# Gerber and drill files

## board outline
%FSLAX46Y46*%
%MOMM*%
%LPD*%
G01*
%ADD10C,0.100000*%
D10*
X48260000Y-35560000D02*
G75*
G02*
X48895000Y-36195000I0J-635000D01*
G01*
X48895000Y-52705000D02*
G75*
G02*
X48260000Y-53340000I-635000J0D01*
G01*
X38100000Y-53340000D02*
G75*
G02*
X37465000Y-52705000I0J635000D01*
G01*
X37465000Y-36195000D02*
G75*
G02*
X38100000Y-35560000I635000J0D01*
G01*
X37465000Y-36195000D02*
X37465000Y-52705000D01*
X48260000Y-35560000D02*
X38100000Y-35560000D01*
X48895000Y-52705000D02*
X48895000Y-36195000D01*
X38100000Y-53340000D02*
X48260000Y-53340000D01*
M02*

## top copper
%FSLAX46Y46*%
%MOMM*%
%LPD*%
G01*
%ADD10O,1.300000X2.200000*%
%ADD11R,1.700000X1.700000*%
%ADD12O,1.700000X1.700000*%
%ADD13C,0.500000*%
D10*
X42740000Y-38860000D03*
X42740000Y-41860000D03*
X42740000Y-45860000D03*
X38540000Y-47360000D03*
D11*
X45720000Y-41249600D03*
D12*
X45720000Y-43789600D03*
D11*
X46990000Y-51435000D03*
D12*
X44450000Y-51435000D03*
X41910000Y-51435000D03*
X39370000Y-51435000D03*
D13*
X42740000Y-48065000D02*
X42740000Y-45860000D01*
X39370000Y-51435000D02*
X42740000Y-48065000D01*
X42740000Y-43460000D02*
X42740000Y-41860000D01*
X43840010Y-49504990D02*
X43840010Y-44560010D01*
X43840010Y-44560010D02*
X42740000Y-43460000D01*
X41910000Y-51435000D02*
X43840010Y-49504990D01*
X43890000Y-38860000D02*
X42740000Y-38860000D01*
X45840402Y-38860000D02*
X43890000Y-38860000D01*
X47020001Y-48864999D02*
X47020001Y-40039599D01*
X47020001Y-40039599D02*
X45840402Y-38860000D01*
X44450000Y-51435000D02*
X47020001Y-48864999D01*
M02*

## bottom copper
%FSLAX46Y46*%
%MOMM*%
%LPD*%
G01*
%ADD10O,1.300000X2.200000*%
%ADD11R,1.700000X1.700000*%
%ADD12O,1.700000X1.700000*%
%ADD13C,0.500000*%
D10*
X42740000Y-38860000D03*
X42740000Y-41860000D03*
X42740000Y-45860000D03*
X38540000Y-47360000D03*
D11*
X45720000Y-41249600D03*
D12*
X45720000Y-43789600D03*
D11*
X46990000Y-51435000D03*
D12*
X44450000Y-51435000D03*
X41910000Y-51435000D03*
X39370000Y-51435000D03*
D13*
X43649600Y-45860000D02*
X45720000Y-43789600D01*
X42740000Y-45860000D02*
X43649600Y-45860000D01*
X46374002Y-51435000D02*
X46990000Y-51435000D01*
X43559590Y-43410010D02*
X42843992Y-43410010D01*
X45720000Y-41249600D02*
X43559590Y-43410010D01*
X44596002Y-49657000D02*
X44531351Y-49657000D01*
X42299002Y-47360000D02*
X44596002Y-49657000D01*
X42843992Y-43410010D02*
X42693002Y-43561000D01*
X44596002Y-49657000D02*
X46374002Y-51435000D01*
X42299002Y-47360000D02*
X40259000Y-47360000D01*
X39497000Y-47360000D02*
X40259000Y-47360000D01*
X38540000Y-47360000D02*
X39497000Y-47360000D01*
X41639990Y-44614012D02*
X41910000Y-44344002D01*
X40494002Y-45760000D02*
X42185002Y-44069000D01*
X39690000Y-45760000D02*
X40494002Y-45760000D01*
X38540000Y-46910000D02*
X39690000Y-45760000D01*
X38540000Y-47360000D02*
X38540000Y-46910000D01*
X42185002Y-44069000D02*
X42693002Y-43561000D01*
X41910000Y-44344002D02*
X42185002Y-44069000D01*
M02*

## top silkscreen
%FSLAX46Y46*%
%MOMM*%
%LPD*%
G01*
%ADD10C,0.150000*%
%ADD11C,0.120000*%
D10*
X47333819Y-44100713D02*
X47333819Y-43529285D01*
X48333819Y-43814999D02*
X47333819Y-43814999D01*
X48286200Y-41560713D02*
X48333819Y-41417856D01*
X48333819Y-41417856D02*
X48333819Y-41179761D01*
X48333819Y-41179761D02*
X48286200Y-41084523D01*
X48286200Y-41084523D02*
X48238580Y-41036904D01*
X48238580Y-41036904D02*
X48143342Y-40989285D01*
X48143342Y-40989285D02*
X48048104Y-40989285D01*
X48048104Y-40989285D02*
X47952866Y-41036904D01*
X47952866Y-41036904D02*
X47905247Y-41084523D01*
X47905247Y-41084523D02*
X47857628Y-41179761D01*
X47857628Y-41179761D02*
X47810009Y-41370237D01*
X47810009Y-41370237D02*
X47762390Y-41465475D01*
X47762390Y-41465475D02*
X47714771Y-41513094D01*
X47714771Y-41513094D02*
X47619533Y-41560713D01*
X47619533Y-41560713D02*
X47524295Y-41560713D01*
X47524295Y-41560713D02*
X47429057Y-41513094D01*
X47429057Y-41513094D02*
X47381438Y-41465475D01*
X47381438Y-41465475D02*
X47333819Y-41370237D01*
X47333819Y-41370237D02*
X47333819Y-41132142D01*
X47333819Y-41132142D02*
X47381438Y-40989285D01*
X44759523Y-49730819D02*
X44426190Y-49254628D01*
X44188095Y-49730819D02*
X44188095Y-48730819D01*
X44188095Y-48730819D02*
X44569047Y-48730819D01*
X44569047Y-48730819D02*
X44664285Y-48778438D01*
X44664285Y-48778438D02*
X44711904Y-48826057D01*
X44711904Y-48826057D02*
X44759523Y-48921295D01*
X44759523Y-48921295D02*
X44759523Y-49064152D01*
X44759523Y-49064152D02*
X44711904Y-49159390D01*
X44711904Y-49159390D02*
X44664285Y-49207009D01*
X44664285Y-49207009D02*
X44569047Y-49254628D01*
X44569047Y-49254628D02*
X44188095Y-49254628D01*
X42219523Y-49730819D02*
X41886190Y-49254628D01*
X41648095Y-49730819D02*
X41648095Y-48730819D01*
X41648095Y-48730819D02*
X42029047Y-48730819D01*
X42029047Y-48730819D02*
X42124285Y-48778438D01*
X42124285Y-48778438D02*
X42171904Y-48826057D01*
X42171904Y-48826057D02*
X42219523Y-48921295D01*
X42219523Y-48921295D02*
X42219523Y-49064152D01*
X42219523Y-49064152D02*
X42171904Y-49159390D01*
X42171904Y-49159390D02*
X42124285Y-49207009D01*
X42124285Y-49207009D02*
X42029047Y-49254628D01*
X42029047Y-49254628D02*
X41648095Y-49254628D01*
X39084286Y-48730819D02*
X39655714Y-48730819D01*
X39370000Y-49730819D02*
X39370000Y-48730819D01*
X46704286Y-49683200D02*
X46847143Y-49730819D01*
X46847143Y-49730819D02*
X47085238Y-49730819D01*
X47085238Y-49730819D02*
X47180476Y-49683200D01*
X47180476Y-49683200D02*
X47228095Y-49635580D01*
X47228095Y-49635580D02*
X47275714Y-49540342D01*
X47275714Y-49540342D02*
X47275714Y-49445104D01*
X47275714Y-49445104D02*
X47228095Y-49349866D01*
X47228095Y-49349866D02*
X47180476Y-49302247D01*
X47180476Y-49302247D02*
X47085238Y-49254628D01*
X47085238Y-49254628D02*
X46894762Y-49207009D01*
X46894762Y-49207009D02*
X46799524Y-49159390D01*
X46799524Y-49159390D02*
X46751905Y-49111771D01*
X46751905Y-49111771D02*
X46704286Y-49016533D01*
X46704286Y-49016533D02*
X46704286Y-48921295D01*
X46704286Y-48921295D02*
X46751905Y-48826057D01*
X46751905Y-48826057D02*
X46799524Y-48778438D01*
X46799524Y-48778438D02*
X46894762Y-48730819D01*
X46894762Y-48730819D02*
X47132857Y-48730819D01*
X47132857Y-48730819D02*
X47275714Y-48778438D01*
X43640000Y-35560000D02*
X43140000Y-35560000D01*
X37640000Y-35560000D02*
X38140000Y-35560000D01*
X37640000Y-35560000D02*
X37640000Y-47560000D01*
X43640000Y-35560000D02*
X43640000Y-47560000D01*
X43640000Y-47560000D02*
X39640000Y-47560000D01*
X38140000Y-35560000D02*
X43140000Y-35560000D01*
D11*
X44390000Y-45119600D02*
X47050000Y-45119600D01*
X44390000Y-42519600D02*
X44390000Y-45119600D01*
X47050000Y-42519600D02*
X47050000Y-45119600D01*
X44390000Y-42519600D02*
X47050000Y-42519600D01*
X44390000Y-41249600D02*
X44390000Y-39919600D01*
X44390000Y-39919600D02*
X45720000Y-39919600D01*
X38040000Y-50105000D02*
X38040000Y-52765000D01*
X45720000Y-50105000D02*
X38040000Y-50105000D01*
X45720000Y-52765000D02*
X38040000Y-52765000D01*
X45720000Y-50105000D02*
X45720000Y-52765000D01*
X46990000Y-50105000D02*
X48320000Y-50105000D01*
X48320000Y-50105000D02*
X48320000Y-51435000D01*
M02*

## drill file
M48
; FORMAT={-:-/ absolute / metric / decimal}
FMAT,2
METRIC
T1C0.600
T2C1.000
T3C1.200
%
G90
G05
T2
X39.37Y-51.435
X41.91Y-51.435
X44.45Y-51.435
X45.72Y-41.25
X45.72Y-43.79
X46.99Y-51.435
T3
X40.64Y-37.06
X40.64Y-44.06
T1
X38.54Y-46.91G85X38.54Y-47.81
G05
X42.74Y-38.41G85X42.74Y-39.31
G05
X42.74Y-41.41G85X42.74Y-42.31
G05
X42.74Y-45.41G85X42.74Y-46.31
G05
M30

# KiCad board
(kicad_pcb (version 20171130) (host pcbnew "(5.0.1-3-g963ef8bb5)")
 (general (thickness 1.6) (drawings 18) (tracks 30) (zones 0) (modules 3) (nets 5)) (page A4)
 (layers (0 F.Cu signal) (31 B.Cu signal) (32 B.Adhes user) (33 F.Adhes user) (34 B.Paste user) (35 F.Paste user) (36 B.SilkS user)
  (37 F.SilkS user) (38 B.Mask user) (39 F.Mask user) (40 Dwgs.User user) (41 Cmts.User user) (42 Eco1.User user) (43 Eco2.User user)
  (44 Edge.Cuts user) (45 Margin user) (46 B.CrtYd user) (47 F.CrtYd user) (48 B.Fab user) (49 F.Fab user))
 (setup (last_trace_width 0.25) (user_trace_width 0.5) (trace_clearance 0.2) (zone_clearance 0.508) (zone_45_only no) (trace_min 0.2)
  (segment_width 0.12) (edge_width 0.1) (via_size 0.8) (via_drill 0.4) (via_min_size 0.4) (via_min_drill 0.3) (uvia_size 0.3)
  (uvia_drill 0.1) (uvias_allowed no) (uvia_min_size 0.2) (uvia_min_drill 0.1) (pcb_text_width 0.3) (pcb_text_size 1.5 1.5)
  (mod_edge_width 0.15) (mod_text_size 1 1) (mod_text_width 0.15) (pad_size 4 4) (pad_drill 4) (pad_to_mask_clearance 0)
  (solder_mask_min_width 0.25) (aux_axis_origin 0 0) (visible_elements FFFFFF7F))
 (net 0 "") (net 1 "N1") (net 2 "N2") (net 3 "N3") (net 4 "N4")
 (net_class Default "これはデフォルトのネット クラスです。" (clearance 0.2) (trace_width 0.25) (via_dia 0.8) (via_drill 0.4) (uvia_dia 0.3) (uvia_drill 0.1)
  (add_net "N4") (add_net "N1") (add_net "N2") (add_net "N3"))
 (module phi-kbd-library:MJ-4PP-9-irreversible (layer F.Cu) (at 40.64 35.56 270)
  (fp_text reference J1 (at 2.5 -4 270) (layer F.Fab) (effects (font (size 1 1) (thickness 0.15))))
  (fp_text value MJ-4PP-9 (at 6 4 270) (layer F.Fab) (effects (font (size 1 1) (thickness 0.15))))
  (fp_line (start 0 -3) (end 0 -2.5) (layer F.SilkS) (width 0.15))
  (fp_line (start 0 3) (end 0 2.5) (layer F.SilkS) (width 0.15))
  (fp_line (start 0 3) (end 12 3) (layer F.SilkS) (width 0.15))
  (fp_line (start 0 -3) (end 12 -3) (layer F.SilkS) (width 0.15))
  (fp_line (start 12 -3) (end 12 1) (layer F.SilkS) (width 0.15))
  (fp_line (start 0 2.5) (end 0 -2.5) (layer F.SilkS) (width 0.15))
  (pad "" np_thru_hole circle (at 1.5 0 270) (size 1.2 1.2) (drill 1.2) (layers *.Cu *.Mask))
  (pad "" np_thru_hole circle (at 8.5 0 270) (size 1.2 1.2) (drill 1.2) (layers *.Cu *.Mask))
  (pad B thru_hole oval (at 3.3 -2.1 270) (size 2.2 1.3) (drill oval 1.5 0.6) (layers *.Cu *.Mask) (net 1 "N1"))
  (pad C thru_hole oval (at 6.3 -2.1 270) (size 2.2 1.3) (drill oval 1.5 0.6) (layers *.Cu *.Mask) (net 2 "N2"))
  (pad D thru_hole oval (at 10.3 -2.1 270) (size 2.2 1.3) (drill oval 1.5 0.6) (layers *.Cu *.Mask) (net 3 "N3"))
  (pad A thru_hole oval (at 11.8 2.1 270) (size 2.2 1.3) (drill oval 1.5 0.6) (layers *.Cu *.Mask) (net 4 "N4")))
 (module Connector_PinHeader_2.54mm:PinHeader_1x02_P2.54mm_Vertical (layer F.Cu) (at 45.72 41.2496)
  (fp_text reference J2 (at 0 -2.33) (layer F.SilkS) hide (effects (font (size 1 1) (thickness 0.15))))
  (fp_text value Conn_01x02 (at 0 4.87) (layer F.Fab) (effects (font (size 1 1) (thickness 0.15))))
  (fp_line (start -1.33 3.87) (end 1.33 3.87) (layer F.SilkS) (width 0.12))
  (fp_line (start -1.33 1.27) (end -1.33 3.87) (layer F.SilkS) (width 0.12))
  (fp_line (start 1.33 1.27) (end 1.33 3.87) (layer F.SilkS) (width 0.12))
  (fp_line (start -1.33 1.27) (end 1.33 1.27) (layer F.SilkS) (width 0.12))
  (fp_line (start -1.33 0) (end -1.33 -1.33) (layer F.SilkS) (width 0.12))
  (fp_line (start -1.33 -1.33) (end 0 -1.33) (layer F.SilkS) (width 0.12))
  (pad 1 thru_hole rect (at 0 0) (size 1.7 1.7) (drill 1) (layers *.Cu *.Mask) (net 4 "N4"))
  (pad 2 thru_hole oval (at 0 2.54) (size 1.7 1.7) (drill 1) (layers *.Cu *.Mask) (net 3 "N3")))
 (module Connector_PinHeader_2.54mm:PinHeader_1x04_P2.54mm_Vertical (layer F.Cu) (at 46.99 51.435 270)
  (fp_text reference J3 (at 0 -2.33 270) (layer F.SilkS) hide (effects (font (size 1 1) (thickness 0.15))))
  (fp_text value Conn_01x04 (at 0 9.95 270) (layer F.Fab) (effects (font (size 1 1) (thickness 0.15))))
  (fp_line (start -1.33 8.95) (end 1.33 8.95) (layer F.SilkS) (width 0.12))
  (fp_line (start -1.33 1.27) (end -1.33 8.95) (layer F.SilkS) (width 0.12))
  (fp_line (start 1.33 1.27) (end 1.33 8.95) (layer F.SilkS) (width 0.12))
  (fp_line (start -1.33 1.27) (end 1.33 1.27) (layer F.SilkS) (width 0.12))
  (fp_line (start -1.33 0) (end -1.33 -1.33) (layer F.SilkS) (width 0.12))
  (fp_line (start -1.33 -1.33) (end 0 -1.33) (layer F.SilkS) (width 0.12))
  (pad 1 thru_hole rect (at 0 0 270) (size 1.7 1.7) (drill 1) (layers *.Cu *.Mask) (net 4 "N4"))
  (pad 2 thru_hole oval (at 0 2.54 270) (size 1.7 1.7) (drill 1) (layers *.Cu *.Mask) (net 1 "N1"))
  (pad 3 thru_hole oval (at 0 5.08 270) (size 1.7 1.7) (drill 1) (layers *.Cu *.Mask) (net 2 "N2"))
  (pad 4 thru_hole oval (at 0 7.62 270) (size 1.7 1.7) (drill 1) (layers *.Cu *.Mask) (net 3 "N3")))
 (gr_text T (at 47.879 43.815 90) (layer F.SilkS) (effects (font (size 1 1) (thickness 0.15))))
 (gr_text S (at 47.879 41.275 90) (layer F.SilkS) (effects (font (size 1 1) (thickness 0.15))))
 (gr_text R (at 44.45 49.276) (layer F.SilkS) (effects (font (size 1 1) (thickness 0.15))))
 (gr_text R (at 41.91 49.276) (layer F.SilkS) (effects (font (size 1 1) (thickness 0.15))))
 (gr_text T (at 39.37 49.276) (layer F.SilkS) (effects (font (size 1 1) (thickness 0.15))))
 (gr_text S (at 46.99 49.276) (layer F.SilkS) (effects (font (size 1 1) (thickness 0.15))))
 (gr_arc (start 48.26 36.195) (end 48.895 36.195) (angle -90) (layer Edge.Cuts) (width 0.1))
 (gr_arc (start 48.26 52.705) (end 48.26 53.34) (angle -90) (layer Edge.Cuts) (width 0.1))
 (gr_arc (start 38.1 52.705) (end 37.465 52.705) (angle -90) (layer Edge.Cuts) (width 0.1))
 (gr_arc (start 38.1 36.195) (end 38.1 35.56) (angle -90) (layer Edge.Cuts) (width 0.1))
 (gr_line (start 37.465 36.195) (end 37.465 52.705) (layer Edge.Cuts) (width 0.1))
 (gr_line (start 48.26 35.56) (end 38.1 35.56) (layer Edge.Cuts) (width 0.1))
 (gr_line (start 48.895 52.705) (end 48.895 36.195) (layer Edge.Cuts) (width 0.1))
 (gr_line (start 38.1 53.34) (end 48.26 53.34) (layer Edge.Cuts) (width 0.1))
 (segment (start 43.6496 45.86) (end 45.72 43.7896) (width 0.5) (layer B.Cu) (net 3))
 (segment (start 42.74 45.86) (end 43.6496 45.86) (width 0.5) (layer B.Cu) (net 3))
 (segment (start 42.74 48.065) (end 42.74 45.86) (width 0.5) (layer F.Cu) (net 3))
 (segment (start 39.37 51.435) (end 42.74 48.065) (width 0.5) (layer F.Cu) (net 3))
 (segment (start 42.74 43.46) (end 42.74 41.86) (width 0.5) (layer F.Cu) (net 2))
 (segment (start 43.84001 49.50499) (end 43.84001 44.56001) (width 0.5) (layer F.Cu) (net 2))
 (segment (start 43.84001 44.56001) (end 42.74 43.46) (width 0.5) (layer F.Cu) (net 2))
 (segment (start 41.91 51.435) (end 43.84001 49.50499) (width 0.5) (layer F.Cu) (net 2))
 (segment (start 43.89 38.86) (end 42.74 38.86) (width 0.5) (layer F.Cu) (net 1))
 (segment (start 45.840402 38.86) (end 43.89 38.86) (width 0.5) (layer F.Cu) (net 1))
 (segment (start 47.020001 48.864999) (end 47.020001 40.039599) (width 0.5) (layer F.Cu) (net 1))
 (segment (start 47.020001 40.039599) (end 45.840402 38.86) (width 0.5) (layer F.Cu) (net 1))
 (segment (start 44.45 51.435) (end 47.020001 48.864999) (width 0.5) (layer F.Cu) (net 1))
 (segment (start 46.374002 51.435) (end 46.99 51.435) (width 0.5) (layer B.Cu) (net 4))
 (segment (start 43.55959 43.41001) (end 42.843992 43.41001) (width 0.5) (layer B.Cu) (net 4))
 (segment (start 45.72 41.2496) (end 43.55959 43.41001) (width 0.5) (layer B.Cu) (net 4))
 (segment (start 44.596002 49.657) (end 44.531351 49.657) (width 0.5) (layer B.Cu) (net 4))
 (segment (start 42.299002 47.36) (end 44.596002 49.657) (width 0.5) (layer B.Cu) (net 4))
 (segment (start 42.843992 43.41001) (end 42.693002 43.561) (width 0.5) (layer B.Cu) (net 4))
 (segment (start 44.596002 49.657) (end 46.374002 51.435) (width 0.5) (layer B.Cu) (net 4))
 (segment (start 42.299002 47.36) (end 40.259 47.36) (width 0.5) (layer B.Cu) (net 4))
 (segment (start 39.497 47.36) (end 40.259 47.36) (width 0.5) (layer B.Cu) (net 4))
 (segment (start 38.54 47.36) (end 39.497 47.36) (width 0.5) (layer B.Cu) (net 4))
 (segment (start 41.63999 44.614012) (end 41.91 44.344002) (width 0.5) (layer B.Cu) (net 4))
 (segment (start 40.494002 45.76) (end 42.185002 44.069) (width 0.5) (layer B.Cu) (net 4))
 (segment (start 39.69 45.76) (end 40.494002 45.76) (width 0.5) (layer B.Cu) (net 4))
 (segment (start 38.54 46.91) (end 39.69 45.76) (width 0.5) (layer B.Cu) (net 4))
 (segment (start 38.54 47.36) (end 38.54 46.91) (width 0.5) (layer B.Cu) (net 4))
 (segment (start 42.185002 44.069) (end 42.693002 43.561) (width 0.5) (layer B.Cu) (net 4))
 (segment (start 41.91 44.344002) (end 42.185002 44.069) (width 0.5) (layer B.Cu) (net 4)))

